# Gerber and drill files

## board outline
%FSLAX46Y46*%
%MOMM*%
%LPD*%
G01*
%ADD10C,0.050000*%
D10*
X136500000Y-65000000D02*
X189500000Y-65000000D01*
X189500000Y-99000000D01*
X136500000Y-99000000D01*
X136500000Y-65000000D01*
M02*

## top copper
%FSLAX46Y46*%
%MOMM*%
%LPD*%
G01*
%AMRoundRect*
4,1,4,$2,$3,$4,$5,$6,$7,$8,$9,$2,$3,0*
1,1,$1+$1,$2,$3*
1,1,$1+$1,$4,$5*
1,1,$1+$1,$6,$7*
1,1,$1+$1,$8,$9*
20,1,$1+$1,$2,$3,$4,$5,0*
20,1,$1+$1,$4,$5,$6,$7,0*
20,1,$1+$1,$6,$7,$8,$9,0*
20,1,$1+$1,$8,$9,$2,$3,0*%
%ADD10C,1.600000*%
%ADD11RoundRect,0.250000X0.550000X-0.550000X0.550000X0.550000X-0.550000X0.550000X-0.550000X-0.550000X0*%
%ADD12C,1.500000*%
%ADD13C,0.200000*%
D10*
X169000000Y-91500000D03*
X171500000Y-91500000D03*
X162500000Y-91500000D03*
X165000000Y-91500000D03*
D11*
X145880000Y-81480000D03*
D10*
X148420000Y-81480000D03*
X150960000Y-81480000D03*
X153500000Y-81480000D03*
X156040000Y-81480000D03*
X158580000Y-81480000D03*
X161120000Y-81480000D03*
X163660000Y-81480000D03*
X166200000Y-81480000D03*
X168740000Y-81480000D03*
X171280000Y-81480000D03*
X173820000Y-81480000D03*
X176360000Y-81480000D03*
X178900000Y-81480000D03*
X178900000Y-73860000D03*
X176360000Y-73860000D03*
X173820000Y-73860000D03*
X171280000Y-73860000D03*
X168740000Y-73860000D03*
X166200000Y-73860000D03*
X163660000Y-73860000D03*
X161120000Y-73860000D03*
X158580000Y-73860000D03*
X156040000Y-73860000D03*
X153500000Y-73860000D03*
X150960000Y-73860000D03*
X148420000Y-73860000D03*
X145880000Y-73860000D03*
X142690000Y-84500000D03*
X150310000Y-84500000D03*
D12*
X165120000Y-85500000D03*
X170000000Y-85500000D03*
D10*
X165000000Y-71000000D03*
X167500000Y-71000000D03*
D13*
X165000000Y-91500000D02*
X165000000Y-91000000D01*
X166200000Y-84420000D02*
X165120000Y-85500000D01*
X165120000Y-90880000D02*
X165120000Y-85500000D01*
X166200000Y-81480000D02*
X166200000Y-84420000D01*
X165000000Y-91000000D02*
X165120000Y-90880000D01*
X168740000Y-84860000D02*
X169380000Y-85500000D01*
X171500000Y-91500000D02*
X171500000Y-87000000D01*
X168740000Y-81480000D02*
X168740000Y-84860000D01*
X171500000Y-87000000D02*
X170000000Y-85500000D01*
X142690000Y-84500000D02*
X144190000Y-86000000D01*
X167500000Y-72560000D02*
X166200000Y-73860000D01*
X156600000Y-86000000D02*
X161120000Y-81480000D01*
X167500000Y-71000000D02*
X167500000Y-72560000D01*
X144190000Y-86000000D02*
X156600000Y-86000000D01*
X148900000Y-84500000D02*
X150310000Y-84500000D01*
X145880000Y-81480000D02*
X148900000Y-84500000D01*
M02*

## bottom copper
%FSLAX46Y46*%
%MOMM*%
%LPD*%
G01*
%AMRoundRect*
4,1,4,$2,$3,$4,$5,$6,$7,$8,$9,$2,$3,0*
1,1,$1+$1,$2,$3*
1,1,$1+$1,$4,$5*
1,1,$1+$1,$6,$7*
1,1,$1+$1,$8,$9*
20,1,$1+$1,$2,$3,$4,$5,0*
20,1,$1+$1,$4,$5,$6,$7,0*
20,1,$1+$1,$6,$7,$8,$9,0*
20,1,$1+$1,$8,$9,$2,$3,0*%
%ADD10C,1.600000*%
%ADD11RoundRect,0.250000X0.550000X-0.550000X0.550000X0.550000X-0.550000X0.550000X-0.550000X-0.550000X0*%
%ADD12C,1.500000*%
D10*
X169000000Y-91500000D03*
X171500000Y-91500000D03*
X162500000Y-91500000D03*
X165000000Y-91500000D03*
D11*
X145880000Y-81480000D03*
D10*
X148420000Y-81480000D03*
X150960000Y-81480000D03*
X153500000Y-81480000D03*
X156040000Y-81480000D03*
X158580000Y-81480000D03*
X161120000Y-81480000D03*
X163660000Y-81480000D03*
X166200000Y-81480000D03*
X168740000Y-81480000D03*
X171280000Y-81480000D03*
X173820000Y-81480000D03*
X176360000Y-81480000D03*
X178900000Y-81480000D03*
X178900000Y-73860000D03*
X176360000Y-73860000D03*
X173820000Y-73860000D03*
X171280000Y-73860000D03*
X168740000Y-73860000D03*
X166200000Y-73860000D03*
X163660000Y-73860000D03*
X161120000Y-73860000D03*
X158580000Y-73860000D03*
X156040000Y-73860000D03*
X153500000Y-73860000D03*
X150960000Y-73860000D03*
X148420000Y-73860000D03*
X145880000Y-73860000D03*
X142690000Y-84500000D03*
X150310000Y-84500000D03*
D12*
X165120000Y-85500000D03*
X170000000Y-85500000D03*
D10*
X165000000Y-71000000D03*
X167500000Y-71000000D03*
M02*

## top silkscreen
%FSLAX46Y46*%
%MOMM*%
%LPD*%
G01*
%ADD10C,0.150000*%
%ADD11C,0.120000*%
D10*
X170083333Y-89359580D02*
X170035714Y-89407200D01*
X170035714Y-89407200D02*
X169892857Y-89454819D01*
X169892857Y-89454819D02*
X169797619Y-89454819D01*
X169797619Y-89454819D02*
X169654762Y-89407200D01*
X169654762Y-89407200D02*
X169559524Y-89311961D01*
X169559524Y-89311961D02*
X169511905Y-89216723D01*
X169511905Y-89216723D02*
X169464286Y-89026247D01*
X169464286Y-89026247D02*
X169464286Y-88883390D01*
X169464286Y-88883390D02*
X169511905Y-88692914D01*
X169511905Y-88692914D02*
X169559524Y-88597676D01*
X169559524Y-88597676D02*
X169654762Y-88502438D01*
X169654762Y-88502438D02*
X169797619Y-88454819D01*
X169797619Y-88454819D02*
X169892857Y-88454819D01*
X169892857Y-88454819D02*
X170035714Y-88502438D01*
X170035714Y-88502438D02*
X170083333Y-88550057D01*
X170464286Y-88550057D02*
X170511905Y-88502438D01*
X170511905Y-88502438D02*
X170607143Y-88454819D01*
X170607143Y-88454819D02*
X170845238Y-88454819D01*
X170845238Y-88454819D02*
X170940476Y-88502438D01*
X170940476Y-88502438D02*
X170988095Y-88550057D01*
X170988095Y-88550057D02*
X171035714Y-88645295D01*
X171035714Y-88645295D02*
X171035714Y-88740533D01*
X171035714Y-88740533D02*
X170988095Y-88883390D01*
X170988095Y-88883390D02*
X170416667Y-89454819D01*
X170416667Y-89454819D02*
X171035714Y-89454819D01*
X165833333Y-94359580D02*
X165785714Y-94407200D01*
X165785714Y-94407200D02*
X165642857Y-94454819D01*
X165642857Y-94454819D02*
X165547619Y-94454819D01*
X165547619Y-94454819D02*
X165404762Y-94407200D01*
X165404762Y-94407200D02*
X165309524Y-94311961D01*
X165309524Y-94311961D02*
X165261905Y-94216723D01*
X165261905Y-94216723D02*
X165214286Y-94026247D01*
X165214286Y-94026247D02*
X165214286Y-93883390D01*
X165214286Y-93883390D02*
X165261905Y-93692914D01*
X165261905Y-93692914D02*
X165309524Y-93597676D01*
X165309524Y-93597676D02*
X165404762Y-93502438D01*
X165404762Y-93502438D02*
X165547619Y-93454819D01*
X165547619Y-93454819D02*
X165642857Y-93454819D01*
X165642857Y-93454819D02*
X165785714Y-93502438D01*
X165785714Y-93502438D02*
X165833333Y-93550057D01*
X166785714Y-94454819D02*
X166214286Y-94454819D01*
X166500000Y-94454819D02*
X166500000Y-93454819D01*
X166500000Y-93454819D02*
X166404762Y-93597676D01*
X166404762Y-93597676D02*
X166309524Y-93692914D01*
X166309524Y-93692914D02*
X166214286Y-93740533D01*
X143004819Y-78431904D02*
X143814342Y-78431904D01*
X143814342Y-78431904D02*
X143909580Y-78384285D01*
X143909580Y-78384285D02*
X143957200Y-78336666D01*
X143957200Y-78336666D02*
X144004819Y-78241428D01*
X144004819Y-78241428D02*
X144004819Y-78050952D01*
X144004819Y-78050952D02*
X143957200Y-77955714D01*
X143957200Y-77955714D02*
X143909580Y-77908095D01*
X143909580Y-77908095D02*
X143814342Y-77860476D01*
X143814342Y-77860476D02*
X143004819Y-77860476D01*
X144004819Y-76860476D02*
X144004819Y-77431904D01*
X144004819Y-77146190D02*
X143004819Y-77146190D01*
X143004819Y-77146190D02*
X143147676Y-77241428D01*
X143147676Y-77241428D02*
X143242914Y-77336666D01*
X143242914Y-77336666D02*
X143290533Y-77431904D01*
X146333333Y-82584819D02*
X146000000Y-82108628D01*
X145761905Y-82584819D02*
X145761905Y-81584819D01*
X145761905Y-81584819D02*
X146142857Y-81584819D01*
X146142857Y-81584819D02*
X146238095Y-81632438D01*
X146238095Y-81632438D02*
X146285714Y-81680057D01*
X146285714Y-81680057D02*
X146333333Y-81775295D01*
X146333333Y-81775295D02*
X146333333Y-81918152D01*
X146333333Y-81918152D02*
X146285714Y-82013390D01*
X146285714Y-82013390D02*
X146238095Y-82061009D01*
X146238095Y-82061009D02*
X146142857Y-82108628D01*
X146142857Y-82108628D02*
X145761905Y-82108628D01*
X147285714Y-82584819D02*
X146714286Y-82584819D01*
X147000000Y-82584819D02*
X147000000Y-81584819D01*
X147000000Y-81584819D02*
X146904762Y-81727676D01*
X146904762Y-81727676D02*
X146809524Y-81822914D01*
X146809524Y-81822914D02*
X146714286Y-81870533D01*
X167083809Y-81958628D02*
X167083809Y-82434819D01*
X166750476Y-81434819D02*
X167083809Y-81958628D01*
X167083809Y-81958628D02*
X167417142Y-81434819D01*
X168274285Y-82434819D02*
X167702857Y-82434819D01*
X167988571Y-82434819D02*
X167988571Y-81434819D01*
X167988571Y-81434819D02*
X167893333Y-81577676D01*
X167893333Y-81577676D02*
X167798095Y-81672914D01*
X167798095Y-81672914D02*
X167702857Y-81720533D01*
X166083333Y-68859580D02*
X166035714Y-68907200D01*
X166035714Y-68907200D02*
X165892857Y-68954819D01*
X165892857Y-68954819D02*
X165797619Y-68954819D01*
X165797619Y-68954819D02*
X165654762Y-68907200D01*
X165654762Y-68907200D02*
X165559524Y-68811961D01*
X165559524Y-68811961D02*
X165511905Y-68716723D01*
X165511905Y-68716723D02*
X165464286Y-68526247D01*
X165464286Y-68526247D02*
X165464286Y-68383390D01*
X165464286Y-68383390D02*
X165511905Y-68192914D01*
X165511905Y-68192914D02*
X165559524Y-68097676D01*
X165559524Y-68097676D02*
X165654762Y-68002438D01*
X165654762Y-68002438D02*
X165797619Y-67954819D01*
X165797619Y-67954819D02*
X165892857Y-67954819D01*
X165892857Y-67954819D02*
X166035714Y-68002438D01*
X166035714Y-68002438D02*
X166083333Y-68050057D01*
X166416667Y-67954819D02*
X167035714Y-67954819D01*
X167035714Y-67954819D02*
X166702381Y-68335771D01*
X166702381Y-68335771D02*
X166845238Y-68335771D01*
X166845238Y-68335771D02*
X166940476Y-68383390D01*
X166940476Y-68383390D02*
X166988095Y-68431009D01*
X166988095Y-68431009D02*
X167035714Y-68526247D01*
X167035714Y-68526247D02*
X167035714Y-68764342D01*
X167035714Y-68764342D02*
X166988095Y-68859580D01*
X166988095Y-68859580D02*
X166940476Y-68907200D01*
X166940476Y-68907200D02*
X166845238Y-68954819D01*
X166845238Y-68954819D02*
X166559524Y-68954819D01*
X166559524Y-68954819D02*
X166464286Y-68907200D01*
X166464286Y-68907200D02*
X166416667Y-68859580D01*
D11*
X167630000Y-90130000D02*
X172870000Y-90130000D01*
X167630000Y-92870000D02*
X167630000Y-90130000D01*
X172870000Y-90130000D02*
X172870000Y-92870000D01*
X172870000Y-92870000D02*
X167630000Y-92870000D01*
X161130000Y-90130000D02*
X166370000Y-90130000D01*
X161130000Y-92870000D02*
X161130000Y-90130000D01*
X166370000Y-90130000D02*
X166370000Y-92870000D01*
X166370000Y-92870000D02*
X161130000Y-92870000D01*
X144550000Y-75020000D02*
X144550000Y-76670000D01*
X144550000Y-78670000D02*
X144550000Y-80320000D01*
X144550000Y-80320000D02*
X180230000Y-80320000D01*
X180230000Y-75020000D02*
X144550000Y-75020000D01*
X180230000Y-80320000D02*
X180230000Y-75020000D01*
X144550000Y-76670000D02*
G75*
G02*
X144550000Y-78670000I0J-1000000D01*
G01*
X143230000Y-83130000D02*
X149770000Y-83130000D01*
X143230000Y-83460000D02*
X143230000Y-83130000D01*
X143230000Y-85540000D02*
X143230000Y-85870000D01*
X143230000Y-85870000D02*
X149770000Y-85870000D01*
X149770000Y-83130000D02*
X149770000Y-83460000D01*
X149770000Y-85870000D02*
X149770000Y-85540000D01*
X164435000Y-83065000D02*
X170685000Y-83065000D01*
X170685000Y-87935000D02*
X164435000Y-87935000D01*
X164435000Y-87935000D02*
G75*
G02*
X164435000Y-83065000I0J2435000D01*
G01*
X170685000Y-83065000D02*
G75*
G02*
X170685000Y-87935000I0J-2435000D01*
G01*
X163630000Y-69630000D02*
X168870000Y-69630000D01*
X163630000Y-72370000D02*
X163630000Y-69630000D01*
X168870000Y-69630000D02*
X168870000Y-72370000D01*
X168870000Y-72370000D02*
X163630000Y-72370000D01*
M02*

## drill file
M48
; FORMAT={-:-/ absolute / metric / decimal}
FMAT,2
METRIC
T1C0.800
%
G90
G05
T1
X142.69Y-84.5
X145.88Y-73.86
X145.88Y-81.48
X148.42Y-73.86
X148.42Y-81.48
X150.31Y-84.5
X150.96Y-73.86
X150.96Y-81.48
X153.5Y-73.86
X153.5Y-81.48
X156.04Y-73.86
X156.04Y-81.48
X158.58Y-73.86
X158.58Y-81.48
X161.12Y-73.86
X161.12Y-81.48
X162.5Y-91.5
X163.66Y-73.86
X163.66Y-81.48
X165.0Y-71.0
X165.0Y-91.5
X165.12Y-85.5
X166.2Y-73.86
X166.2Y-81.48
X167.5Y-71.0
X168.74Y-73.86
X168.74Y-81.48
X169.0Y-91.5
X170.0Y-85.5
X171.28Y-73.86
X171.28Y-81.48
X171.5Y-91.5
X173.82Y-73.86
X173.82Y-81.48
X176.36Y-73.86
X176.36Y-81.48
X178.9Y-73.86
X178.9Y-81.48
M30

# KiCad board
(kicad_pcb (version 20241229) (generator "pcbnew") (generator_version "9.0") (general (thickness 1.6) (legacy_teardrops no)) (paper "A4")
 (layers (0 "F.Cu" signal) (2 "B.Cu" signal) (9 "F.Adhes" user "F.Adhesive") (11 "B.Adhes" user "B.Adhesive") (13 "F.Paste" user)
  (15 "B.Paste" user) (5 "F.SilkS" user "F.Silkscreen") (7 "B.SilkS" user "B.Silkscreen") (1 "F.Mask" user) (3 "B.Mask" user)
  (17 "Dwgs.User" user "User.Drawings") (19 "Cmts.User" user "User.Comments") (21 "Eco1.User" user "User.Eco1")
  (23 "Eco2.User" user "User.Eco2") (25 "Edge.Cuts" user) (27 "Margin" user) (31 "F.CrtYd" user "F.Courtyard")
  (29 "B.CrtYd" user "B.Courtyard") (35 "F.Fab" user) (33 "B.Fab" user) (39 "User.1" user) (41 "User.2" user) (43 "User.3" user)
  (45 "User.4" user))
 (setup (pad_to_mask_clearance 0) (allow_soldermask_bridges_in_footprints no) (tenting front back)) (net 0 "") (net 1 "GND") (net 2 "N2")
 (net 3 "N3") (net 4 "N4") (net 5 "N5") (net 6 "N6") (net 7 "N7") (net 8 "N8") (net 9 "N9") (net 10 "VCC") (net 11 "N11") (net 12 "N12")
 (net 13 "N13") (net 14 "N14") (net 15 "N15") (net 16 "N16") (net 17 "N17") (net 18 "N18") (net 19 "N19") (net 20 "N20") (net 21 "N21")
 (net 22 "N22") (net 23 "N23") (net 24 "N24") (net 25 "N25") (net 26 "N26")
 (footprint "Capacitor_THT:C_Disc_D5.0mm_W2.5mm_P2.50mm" (layer "F.Cu") (at 169 91.5)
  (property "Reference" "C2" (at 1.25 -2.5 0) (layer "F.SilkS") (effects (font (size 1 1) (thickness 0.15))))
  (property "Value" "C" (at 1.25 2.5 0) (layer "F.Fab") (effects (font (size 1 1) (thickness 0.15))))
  (fp_line (start -1.37 -1.37) (end 3.87 -1.37) (stroke (width 0.12) (type solid)) (layer "F.SilkS"))
  (fp_line (start -1.37 1.37) (end -1.37 -1.37) (stroke (width 0.12) (type solid)) (layer "F.SilkS"))
  (fp_line (start 3.87 -1.37) (end 3.87 1.37) (stroke (width 0.12) (type solid)) (layer "F.SilkS"))
  (fp_line (start 3.87 1.37) (end -1.37 1.37) (stroke (width 0.12) (type solid)) (layer "F.SilkS"))
  (pad "1" thru_hole circle (at 0 0) (size 1.6 1.6) (drill 0.8) (layers "*.Cu" "*.Mask") (remove_unused_layers no) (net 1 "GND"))
  (pad "2" thru_hole circle (at 2.5 0) (size 1.6 1.6) (drill 0.8) (layers "*.Cu" "*.Mask") (remove_unused_layers no) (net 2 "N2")))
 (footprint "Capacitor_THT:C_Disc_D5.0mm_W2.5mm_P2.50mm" (layer "F.Cu") (at 162.5 91.5)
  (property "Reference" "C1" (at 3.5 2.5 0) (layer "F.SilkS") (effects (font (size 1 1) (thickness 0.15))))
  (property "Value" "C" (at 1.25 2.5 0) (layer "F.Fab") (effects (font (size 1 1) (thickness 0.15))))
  (fp_line (start -1.37 -1.37) (end 3.87 -1.37) (stroke (width 0.12) (type solid)) (layer "F.SilkS"))
  (fp_line (start -1.37 1.37) (end -1.37 -1.37) (stroke (width 0.12) (type solid)) (layer "F.SilkS"))
  (fp_line (start 3.87 -1.37) (end 3.87 1.37) (stroke (width 0.12) (type solid)) (layer "F.SilkS"))
  (fp_line (start 3.87 1.37) (end -1.37 1.37) (stroke (width 0.12) (type solid)) (layer "F.SilkS"))
  (pad "1" thru_hole circle (at 0 0) (size 1.6 1.6) (drill 0.8) (layers "*.Cu" "*.Mask") (remove_unused_layers no) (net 1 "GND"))
  (pad "2" thru_hole circle (at 2.5 0) (size 1.6 1.6) (drill 0.8) (layers "*.Cu" "*.Mask") (remove_unused_layers no) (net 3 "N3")))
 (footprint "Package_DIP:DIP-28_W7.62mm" (layer "F.Cu") (at 145.88 81.48 90)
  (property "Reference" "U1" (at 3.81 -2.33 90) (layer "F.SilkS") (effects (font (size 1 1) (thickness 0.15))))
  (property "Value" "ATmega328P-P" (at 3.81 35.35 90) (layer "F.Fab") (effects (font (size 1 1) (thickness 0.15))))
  (fp_line (start 6.46 -1.33) (end 4.81 -1.33) (stroke (width 0.12) (type solid)) (layer "F.SilkS"))
  (fp_line (start 2.81 -1.33) (end 1.16 -1.33) (stroke (width 0.12) (type solid)) (layer "F.SilkS"))
  (fp_line (start 1.16 -1.33) (end 1.16 34.35) (stroke (width 0.12) (type solid)) (layer "F.SilkS"))
  (fp_line (start 6.46 34.35) (end 6.46 -1.33) (stroke (width 0.12) (type solid)) (layer "F.SilkS"))
  (fp_line (start 1.16 34.35) (end 6.46 34.35) (stroke (width 0.12) (type solid)) (layer "F.SilkS"))
  (fp_arc (start 4.81 -1.33) (mid 3.81 -0.33) (end 2.81 -1.33) (stroke (width 0.12) (type solid)) (layer "F.SilkS"))
  (pad "1" thru_hole roundrect (at 0 0 90) (size 1.6 1.6) (drill 0.8) (layers "*.Cu" "*.Mask") (remove_unused_layers no)
   (roundrect_rratio 0.15625) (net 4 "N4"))
  (pad "2" thru_hole circle (at 0 2.54 90) (size 1.6 1.6) (drill 0.8) (layers "*.Cu" "*.Mask") (remove_unused_layers no) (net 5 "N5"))
  (pad "3" thru_hole circle (at 0 5.08 90) (size 1.6 1.6) (drill 0.8) (layers "*.Cu" "*.Mask") (remove_unused_layers no) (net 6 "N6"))
  (pad "4" thru_hole circle (at 0 7.62 90) (size 1.6 1.6) (drill 0.8) (layers "*.Cu" "*.Mask") (remove_unused_layers no) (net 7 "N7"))
  (pad "5" thru_hole circle (at 0 10.16 90) (size 1.6 1.6) (drill 0.8) (layers "*.Cu" "*.Mask") (remove_unused_layers no) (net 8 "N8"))
  (pad "6" thru_hole circle (at 0 12.7 90) (size 1.6 1.6) (drill 0.8) (layers "*.Cu" "*.Mask") (remove_unused_layers no) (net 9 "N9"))
  (pad "7" thru_hole circle (at 0 15.24 90) (size 1.6 1.6) (drill 0.8) (layers "*.Cu" "*.Mask") (remove_unused_layers no) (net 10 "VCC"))
  (pad "8" thru_hole circle (at 0 17.78 90) (size 1.6 1.6) (drill 0.8) (layers "*.Cu" "*.Mask") (remove_unused_layers no) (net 1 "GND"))
  (pad "9" thru_hole circle (at 0 20.32 90) (size 1.6 1.6) (drill 0.8) (layers "*.Cu" "*.Mask") (remove_unused_layers no) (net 3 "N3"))
  (pad "10" thru_hole circle (at 0 22.86 90) (size 1.6 1.6) (drill 0.8) (layers "*.Cu" "*.Mask") (remove_unused_layers no) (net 2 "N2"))
  (pad "11" thru_hole circle (at 0 25.4 90) (size 1.6 1.6) (drill 0.8) (layers "*.Cu" "*.Mask") (remove_unused_layers no) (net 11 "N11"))
  (pad "12" thru_hole circle (at 0 27.94 90) (size 1.6 1.6) (drill 0.8) (layers "*.Cu" "*.Mask") (remove_unused_layers no) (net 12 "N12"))
  (pad "13" thru_hole circle (at 0 30.48 90) (size 1.6 1.6) (drill 0.8) (layers "*.Cu" "*.Mask") (remove_unused_layers no) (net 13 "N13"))
  (pad "14" thru_hole circle (at 0 33.02 90) (size 1.6 1.6) (drill 0.8) (layers "*.Cu" "*.Mask") (remove_unused_layers no) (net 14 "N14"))
  (pad "15" thru_hole circle (at 7.62 33.02 90) (size 1.6 1.6) (drill 0.8) (layers "*.Cu" "*.Mask") (remove_unused_layers no) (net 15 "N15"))
  (pad "16" thru_hole circle (at 7.62 30.48 90) (size 1.6 1.6) (drill 0.8) (layers "*.Cu" "*.Mask") (remove_unused_layers no) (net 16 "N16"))
  (pad "17" thru_hole circle (at 7.62 27.94 90) (size 1.6 1.6) (drill 0.8) (layers "*.Cu" "*.Mask") (remove_unused_layers no) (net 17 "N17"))
  (pad "18" thru_hole circle (at 7.62 25.4 90) (size 1.6 1.6) (drill 0.8) (layers "*.Cu" "*.Mask") (remove_unused_layers no) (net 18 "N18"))
  (pad "19" thru_hole circle (at 7.62 22.86 90) (size 1.6 1.6) (drill 0.8) (layers "*.Cu" "*.Mask") (remove_unused_layers no) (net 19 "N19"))
  (pad "20" thru_hole circle (at 7.62 20.32 90) (size 1.6 1.6) (drill 0.8) (layers "*.Cu" "*.Mask") (remove_unused_layers no) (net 10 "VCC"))
  (pad "21" thru_hole circle (at 7.62 17.78 90) (size 1.6 1.6) (drill 0.8) (layers "*.Cu" "*.Mask") (remove_unused_layers no) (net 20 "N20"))
  (pad "22" thru_hole circle (at 7.62 15.24 90) (size 1.6 1.6) (drill 0.8) (layers "*.Cu" "*.Mask") (remove_unused_layers no) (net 1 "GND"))
  (pad "23" thru_hole circle (at 7.62 12.7 90) (size 1.6 1.6) (drill 0.8) (layers "*.Cu" "*.Mask") (remove_unused_layers no) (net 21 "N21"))
  (pad "24" thru_hole circle (at 7.62 10.16 90) (size 1.6 1.6) (drill 0.8) (layers "*.Cu" "*.Mask") (remove_unused_layers no) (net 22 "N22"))
  (pad "25" thru_hole circle (at 7.62 7.62 90) (size 1.6 1.6) (drill 0.8) (layers "*.Cu" "*.Mask") (remove_unused_layers no) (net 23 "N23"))
  (pad "26" thru_hole circle (at 7.62 5.08 90) (size 1.6 1.6) (drill 0.8) (layers "*.Cu" "*.Mask") (remove_unused_layers no) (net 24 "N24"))
  (pad "27" thru_hole circle (at 7.62 2.54 90) (size 1.6 1.6) (drill 0.8) (layers "*.Cu" "*.Mask") (remove_unused_layers no) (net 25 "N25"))
  (pad "28" thru_hole circle (at 7.62 0 90) (size 1.6 1.6) (drill 0.8) (layers "*.Cu" "*.Mask") (remove_unused_layers no) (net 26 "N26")))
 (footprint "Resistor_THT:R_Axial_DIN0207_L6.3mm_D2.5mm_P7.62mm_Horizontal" (layer "F.Cu") (at 142.69 84.5)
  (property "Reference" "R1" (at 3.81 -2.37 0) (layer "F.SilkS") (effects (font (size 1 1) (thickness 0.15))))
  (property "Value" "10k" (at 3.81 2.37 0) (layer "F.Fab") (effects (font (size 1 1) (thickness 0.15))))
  (fp_line (start 0.54 -1.37) (end 7.08 -1.37) (stroke (width 0.12) (type solid)) (layer "F.SilkS"))
  (fp_line (start 0.54 -1.04) (end 0.54 -1.37) (stroke (width 0.12) (type solid)) (layer "F.SilkS"))
  (fp_line (start 0.54 1.04) (end 0.54 1.37) (stroke (width 0.12) (type solid)) (layer "F.SilkS"))
  (fp_line (start 0.54 1.37) (end 7.08 1.37) (stroke (width 0.12) (type solid)) (layer "F.SilkS"))
  (fp_line (start 7.08 -1.37) (end 7.08 -1.04) (stroke (width 0.12) (type solid)) (layer "F.SilkS"))
  (fp_line (start 7.08 1.37) (end 7.08 1.04) (stroke (width 0.12) (type solid)) (layer "F.SilkS"))
  (pad "1" thru_hole circle (at 0 0) (size 1.6 1.6) (drill 0.8) (layers "*.Cu" "*.Mask") (remove_unused_layers no) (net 10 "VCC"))
  (pad "2" thru_hole circle (at 7.62 0) (size 1.6 1.6) (drill 0.8) (layers "*.Cu" "*.Mask") (remove_unused_layers no) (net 4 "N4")))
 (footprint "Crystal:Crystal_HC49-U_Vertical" (layer "F.Cu") (at 165.12 85.5)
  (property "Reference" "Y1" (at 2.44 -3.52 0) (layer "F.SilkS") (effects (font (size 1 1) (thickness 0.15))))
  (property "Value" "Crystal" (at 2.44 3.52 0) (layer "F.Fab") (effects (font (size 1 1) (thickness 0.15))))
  (fp_line (start -0.685 -2.435) (end 5.565 -2.435) (stroke (width 0.12) (type solid)) (layer "F.SilkS"))
  (fp_line (start 5.565 2.435) (end -0.685 2.435) (stroke (width 0.12) (type solid)) (layer "F.SilkS"))
  (fp_arc (start -0.685 2.435) (mid -3.12 0) (end -0.685 -2.435) (stroke (width 0.12) (type solid)) (layer "F.SilkS"))
  (fp_arc (start 5.565 -2.435) (mid 8 0) (end 5.565 2.435) (stroke (width 0.12) (type solid)) (layer "F.SilkS"))
  (pad "1" thru_hole circle (at 0 0) (size 1.5 1.5) (drill 0.8) (layers "*.Cu" "*.Mask") (remove_unused_layers no) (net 3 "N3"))
  (pad "2" thru_hole circle (at 4.88 0) (size 1.5 1.5) (drill 0.8) (layers "*.Cu" "*.Mask") (remove_unused_layers no) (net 2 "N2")))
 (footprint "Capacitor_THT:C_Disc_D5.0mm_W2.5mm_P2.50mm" (layer "F.Cu") (at 165 71)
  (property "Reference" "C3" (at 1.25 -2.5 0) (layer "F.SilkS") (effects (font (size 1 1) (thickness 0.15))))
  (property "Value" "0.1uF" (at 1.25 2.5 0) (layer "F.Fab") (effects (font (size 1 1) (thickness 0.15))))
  (fp_line (start -1.37 -1.37) (end 3.87 -1.37) (stroke (width 0.12) (type solid)) (layer "F.SilkS"))
  (fp_line (start -1.37 1.37) (end -1.37 -1.37) (stroke (width 0.12) (type solid)) (layer "F.SilkS"))
  (fp_line (start 3.87 -1.37) (end 3.87 1.37) (stroke (width 0.12) (type solid)) (layer "F.SilkS"))
  (fp_line (start 3.87 1.37) (end -1.37 1.37) (stroke (width 0.12) (type solid)) (layer "F.SilkS"))
  (pad "1" thru_hole circle (at 0 0) (size 1.6 1.6) (drill 0.8) (layers "*.Cu" "*.Mask") (remove_unused_layers no) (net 1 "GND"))
  (pad "2" thru_hole circle (at 2.5 0) (size 1.6 1.6) (drill 0.8) (layers "*.Cu" "*.Mask") (remove_unused_layers no) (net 10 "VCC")))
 (gr_rect (start 136.5 65) (end 189.5 99) (stroke (width 0.05) (type default)) (fill no) (layer "Edge.Cuts"))
 (segment (start 165 91.5) (end 165 91) (width 0.2) (layer "F.Cu") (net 3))
 (segment (start 166.2 84.42) (end 165.12 85.5) (width 0.2) (layer "F.Cu") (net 3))
 (segment (start 165.12 90.88) (end 165.12 85.5) (width 0.2) (layer "F.Cu") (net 3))
 (segment (start 166.2 81.48) (end 166.2 84.42) (width 0.2) (layer "F.Cu") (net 3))
 (segment (start 165 91) (end 165.12 90.88) (width 0.2) (layer "F.Cu") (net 3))
 (segment (start 168.74 84.86) (end 169.38 85.5) (width 0.2) (layer "F.Cu") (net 2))
 (segment (start 171.5 91.5) (end 171.5 87) (width 0.2) (layer "F.Cu") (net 2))
 (segment (start 168.74 81.48) (end 168.74 84.86) (width 0.2) (layer "F.Cu") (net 2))
 (segment (start 171.5 87) (end 170 85.5) (width 0.2) (layer "F.Cu") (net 2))
 (segment (start 142.69 84.5) (end 144.19 86) (width 0.2) (layer "F.Cu") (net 10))
 (segment (start 167.5 72.56) (end 166.2 73.86) (width 0.2) (layer "F.Cu") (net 10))
 (segment (start 156.6 86) (end 161.12 81.48) (width 0.2) (layer "F.Cu") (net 10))
 (segment (start 167.5 71) (end 167.5 72.56) (width 0.2) (layer "F.Cu") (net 10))
 (segment (start 144.19 86) (end 156.6 86) (width 0.2) (layer "F.Cu") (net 10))
 (segment (start 148.9 84.5) (end 150.31 84.5) (width 0.2) (layer "F.Cu") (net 4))
 (segment (start 145.88 81.48) (end 148.9 84.5) (width 0.2) (layer "F.Cu") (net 4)))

